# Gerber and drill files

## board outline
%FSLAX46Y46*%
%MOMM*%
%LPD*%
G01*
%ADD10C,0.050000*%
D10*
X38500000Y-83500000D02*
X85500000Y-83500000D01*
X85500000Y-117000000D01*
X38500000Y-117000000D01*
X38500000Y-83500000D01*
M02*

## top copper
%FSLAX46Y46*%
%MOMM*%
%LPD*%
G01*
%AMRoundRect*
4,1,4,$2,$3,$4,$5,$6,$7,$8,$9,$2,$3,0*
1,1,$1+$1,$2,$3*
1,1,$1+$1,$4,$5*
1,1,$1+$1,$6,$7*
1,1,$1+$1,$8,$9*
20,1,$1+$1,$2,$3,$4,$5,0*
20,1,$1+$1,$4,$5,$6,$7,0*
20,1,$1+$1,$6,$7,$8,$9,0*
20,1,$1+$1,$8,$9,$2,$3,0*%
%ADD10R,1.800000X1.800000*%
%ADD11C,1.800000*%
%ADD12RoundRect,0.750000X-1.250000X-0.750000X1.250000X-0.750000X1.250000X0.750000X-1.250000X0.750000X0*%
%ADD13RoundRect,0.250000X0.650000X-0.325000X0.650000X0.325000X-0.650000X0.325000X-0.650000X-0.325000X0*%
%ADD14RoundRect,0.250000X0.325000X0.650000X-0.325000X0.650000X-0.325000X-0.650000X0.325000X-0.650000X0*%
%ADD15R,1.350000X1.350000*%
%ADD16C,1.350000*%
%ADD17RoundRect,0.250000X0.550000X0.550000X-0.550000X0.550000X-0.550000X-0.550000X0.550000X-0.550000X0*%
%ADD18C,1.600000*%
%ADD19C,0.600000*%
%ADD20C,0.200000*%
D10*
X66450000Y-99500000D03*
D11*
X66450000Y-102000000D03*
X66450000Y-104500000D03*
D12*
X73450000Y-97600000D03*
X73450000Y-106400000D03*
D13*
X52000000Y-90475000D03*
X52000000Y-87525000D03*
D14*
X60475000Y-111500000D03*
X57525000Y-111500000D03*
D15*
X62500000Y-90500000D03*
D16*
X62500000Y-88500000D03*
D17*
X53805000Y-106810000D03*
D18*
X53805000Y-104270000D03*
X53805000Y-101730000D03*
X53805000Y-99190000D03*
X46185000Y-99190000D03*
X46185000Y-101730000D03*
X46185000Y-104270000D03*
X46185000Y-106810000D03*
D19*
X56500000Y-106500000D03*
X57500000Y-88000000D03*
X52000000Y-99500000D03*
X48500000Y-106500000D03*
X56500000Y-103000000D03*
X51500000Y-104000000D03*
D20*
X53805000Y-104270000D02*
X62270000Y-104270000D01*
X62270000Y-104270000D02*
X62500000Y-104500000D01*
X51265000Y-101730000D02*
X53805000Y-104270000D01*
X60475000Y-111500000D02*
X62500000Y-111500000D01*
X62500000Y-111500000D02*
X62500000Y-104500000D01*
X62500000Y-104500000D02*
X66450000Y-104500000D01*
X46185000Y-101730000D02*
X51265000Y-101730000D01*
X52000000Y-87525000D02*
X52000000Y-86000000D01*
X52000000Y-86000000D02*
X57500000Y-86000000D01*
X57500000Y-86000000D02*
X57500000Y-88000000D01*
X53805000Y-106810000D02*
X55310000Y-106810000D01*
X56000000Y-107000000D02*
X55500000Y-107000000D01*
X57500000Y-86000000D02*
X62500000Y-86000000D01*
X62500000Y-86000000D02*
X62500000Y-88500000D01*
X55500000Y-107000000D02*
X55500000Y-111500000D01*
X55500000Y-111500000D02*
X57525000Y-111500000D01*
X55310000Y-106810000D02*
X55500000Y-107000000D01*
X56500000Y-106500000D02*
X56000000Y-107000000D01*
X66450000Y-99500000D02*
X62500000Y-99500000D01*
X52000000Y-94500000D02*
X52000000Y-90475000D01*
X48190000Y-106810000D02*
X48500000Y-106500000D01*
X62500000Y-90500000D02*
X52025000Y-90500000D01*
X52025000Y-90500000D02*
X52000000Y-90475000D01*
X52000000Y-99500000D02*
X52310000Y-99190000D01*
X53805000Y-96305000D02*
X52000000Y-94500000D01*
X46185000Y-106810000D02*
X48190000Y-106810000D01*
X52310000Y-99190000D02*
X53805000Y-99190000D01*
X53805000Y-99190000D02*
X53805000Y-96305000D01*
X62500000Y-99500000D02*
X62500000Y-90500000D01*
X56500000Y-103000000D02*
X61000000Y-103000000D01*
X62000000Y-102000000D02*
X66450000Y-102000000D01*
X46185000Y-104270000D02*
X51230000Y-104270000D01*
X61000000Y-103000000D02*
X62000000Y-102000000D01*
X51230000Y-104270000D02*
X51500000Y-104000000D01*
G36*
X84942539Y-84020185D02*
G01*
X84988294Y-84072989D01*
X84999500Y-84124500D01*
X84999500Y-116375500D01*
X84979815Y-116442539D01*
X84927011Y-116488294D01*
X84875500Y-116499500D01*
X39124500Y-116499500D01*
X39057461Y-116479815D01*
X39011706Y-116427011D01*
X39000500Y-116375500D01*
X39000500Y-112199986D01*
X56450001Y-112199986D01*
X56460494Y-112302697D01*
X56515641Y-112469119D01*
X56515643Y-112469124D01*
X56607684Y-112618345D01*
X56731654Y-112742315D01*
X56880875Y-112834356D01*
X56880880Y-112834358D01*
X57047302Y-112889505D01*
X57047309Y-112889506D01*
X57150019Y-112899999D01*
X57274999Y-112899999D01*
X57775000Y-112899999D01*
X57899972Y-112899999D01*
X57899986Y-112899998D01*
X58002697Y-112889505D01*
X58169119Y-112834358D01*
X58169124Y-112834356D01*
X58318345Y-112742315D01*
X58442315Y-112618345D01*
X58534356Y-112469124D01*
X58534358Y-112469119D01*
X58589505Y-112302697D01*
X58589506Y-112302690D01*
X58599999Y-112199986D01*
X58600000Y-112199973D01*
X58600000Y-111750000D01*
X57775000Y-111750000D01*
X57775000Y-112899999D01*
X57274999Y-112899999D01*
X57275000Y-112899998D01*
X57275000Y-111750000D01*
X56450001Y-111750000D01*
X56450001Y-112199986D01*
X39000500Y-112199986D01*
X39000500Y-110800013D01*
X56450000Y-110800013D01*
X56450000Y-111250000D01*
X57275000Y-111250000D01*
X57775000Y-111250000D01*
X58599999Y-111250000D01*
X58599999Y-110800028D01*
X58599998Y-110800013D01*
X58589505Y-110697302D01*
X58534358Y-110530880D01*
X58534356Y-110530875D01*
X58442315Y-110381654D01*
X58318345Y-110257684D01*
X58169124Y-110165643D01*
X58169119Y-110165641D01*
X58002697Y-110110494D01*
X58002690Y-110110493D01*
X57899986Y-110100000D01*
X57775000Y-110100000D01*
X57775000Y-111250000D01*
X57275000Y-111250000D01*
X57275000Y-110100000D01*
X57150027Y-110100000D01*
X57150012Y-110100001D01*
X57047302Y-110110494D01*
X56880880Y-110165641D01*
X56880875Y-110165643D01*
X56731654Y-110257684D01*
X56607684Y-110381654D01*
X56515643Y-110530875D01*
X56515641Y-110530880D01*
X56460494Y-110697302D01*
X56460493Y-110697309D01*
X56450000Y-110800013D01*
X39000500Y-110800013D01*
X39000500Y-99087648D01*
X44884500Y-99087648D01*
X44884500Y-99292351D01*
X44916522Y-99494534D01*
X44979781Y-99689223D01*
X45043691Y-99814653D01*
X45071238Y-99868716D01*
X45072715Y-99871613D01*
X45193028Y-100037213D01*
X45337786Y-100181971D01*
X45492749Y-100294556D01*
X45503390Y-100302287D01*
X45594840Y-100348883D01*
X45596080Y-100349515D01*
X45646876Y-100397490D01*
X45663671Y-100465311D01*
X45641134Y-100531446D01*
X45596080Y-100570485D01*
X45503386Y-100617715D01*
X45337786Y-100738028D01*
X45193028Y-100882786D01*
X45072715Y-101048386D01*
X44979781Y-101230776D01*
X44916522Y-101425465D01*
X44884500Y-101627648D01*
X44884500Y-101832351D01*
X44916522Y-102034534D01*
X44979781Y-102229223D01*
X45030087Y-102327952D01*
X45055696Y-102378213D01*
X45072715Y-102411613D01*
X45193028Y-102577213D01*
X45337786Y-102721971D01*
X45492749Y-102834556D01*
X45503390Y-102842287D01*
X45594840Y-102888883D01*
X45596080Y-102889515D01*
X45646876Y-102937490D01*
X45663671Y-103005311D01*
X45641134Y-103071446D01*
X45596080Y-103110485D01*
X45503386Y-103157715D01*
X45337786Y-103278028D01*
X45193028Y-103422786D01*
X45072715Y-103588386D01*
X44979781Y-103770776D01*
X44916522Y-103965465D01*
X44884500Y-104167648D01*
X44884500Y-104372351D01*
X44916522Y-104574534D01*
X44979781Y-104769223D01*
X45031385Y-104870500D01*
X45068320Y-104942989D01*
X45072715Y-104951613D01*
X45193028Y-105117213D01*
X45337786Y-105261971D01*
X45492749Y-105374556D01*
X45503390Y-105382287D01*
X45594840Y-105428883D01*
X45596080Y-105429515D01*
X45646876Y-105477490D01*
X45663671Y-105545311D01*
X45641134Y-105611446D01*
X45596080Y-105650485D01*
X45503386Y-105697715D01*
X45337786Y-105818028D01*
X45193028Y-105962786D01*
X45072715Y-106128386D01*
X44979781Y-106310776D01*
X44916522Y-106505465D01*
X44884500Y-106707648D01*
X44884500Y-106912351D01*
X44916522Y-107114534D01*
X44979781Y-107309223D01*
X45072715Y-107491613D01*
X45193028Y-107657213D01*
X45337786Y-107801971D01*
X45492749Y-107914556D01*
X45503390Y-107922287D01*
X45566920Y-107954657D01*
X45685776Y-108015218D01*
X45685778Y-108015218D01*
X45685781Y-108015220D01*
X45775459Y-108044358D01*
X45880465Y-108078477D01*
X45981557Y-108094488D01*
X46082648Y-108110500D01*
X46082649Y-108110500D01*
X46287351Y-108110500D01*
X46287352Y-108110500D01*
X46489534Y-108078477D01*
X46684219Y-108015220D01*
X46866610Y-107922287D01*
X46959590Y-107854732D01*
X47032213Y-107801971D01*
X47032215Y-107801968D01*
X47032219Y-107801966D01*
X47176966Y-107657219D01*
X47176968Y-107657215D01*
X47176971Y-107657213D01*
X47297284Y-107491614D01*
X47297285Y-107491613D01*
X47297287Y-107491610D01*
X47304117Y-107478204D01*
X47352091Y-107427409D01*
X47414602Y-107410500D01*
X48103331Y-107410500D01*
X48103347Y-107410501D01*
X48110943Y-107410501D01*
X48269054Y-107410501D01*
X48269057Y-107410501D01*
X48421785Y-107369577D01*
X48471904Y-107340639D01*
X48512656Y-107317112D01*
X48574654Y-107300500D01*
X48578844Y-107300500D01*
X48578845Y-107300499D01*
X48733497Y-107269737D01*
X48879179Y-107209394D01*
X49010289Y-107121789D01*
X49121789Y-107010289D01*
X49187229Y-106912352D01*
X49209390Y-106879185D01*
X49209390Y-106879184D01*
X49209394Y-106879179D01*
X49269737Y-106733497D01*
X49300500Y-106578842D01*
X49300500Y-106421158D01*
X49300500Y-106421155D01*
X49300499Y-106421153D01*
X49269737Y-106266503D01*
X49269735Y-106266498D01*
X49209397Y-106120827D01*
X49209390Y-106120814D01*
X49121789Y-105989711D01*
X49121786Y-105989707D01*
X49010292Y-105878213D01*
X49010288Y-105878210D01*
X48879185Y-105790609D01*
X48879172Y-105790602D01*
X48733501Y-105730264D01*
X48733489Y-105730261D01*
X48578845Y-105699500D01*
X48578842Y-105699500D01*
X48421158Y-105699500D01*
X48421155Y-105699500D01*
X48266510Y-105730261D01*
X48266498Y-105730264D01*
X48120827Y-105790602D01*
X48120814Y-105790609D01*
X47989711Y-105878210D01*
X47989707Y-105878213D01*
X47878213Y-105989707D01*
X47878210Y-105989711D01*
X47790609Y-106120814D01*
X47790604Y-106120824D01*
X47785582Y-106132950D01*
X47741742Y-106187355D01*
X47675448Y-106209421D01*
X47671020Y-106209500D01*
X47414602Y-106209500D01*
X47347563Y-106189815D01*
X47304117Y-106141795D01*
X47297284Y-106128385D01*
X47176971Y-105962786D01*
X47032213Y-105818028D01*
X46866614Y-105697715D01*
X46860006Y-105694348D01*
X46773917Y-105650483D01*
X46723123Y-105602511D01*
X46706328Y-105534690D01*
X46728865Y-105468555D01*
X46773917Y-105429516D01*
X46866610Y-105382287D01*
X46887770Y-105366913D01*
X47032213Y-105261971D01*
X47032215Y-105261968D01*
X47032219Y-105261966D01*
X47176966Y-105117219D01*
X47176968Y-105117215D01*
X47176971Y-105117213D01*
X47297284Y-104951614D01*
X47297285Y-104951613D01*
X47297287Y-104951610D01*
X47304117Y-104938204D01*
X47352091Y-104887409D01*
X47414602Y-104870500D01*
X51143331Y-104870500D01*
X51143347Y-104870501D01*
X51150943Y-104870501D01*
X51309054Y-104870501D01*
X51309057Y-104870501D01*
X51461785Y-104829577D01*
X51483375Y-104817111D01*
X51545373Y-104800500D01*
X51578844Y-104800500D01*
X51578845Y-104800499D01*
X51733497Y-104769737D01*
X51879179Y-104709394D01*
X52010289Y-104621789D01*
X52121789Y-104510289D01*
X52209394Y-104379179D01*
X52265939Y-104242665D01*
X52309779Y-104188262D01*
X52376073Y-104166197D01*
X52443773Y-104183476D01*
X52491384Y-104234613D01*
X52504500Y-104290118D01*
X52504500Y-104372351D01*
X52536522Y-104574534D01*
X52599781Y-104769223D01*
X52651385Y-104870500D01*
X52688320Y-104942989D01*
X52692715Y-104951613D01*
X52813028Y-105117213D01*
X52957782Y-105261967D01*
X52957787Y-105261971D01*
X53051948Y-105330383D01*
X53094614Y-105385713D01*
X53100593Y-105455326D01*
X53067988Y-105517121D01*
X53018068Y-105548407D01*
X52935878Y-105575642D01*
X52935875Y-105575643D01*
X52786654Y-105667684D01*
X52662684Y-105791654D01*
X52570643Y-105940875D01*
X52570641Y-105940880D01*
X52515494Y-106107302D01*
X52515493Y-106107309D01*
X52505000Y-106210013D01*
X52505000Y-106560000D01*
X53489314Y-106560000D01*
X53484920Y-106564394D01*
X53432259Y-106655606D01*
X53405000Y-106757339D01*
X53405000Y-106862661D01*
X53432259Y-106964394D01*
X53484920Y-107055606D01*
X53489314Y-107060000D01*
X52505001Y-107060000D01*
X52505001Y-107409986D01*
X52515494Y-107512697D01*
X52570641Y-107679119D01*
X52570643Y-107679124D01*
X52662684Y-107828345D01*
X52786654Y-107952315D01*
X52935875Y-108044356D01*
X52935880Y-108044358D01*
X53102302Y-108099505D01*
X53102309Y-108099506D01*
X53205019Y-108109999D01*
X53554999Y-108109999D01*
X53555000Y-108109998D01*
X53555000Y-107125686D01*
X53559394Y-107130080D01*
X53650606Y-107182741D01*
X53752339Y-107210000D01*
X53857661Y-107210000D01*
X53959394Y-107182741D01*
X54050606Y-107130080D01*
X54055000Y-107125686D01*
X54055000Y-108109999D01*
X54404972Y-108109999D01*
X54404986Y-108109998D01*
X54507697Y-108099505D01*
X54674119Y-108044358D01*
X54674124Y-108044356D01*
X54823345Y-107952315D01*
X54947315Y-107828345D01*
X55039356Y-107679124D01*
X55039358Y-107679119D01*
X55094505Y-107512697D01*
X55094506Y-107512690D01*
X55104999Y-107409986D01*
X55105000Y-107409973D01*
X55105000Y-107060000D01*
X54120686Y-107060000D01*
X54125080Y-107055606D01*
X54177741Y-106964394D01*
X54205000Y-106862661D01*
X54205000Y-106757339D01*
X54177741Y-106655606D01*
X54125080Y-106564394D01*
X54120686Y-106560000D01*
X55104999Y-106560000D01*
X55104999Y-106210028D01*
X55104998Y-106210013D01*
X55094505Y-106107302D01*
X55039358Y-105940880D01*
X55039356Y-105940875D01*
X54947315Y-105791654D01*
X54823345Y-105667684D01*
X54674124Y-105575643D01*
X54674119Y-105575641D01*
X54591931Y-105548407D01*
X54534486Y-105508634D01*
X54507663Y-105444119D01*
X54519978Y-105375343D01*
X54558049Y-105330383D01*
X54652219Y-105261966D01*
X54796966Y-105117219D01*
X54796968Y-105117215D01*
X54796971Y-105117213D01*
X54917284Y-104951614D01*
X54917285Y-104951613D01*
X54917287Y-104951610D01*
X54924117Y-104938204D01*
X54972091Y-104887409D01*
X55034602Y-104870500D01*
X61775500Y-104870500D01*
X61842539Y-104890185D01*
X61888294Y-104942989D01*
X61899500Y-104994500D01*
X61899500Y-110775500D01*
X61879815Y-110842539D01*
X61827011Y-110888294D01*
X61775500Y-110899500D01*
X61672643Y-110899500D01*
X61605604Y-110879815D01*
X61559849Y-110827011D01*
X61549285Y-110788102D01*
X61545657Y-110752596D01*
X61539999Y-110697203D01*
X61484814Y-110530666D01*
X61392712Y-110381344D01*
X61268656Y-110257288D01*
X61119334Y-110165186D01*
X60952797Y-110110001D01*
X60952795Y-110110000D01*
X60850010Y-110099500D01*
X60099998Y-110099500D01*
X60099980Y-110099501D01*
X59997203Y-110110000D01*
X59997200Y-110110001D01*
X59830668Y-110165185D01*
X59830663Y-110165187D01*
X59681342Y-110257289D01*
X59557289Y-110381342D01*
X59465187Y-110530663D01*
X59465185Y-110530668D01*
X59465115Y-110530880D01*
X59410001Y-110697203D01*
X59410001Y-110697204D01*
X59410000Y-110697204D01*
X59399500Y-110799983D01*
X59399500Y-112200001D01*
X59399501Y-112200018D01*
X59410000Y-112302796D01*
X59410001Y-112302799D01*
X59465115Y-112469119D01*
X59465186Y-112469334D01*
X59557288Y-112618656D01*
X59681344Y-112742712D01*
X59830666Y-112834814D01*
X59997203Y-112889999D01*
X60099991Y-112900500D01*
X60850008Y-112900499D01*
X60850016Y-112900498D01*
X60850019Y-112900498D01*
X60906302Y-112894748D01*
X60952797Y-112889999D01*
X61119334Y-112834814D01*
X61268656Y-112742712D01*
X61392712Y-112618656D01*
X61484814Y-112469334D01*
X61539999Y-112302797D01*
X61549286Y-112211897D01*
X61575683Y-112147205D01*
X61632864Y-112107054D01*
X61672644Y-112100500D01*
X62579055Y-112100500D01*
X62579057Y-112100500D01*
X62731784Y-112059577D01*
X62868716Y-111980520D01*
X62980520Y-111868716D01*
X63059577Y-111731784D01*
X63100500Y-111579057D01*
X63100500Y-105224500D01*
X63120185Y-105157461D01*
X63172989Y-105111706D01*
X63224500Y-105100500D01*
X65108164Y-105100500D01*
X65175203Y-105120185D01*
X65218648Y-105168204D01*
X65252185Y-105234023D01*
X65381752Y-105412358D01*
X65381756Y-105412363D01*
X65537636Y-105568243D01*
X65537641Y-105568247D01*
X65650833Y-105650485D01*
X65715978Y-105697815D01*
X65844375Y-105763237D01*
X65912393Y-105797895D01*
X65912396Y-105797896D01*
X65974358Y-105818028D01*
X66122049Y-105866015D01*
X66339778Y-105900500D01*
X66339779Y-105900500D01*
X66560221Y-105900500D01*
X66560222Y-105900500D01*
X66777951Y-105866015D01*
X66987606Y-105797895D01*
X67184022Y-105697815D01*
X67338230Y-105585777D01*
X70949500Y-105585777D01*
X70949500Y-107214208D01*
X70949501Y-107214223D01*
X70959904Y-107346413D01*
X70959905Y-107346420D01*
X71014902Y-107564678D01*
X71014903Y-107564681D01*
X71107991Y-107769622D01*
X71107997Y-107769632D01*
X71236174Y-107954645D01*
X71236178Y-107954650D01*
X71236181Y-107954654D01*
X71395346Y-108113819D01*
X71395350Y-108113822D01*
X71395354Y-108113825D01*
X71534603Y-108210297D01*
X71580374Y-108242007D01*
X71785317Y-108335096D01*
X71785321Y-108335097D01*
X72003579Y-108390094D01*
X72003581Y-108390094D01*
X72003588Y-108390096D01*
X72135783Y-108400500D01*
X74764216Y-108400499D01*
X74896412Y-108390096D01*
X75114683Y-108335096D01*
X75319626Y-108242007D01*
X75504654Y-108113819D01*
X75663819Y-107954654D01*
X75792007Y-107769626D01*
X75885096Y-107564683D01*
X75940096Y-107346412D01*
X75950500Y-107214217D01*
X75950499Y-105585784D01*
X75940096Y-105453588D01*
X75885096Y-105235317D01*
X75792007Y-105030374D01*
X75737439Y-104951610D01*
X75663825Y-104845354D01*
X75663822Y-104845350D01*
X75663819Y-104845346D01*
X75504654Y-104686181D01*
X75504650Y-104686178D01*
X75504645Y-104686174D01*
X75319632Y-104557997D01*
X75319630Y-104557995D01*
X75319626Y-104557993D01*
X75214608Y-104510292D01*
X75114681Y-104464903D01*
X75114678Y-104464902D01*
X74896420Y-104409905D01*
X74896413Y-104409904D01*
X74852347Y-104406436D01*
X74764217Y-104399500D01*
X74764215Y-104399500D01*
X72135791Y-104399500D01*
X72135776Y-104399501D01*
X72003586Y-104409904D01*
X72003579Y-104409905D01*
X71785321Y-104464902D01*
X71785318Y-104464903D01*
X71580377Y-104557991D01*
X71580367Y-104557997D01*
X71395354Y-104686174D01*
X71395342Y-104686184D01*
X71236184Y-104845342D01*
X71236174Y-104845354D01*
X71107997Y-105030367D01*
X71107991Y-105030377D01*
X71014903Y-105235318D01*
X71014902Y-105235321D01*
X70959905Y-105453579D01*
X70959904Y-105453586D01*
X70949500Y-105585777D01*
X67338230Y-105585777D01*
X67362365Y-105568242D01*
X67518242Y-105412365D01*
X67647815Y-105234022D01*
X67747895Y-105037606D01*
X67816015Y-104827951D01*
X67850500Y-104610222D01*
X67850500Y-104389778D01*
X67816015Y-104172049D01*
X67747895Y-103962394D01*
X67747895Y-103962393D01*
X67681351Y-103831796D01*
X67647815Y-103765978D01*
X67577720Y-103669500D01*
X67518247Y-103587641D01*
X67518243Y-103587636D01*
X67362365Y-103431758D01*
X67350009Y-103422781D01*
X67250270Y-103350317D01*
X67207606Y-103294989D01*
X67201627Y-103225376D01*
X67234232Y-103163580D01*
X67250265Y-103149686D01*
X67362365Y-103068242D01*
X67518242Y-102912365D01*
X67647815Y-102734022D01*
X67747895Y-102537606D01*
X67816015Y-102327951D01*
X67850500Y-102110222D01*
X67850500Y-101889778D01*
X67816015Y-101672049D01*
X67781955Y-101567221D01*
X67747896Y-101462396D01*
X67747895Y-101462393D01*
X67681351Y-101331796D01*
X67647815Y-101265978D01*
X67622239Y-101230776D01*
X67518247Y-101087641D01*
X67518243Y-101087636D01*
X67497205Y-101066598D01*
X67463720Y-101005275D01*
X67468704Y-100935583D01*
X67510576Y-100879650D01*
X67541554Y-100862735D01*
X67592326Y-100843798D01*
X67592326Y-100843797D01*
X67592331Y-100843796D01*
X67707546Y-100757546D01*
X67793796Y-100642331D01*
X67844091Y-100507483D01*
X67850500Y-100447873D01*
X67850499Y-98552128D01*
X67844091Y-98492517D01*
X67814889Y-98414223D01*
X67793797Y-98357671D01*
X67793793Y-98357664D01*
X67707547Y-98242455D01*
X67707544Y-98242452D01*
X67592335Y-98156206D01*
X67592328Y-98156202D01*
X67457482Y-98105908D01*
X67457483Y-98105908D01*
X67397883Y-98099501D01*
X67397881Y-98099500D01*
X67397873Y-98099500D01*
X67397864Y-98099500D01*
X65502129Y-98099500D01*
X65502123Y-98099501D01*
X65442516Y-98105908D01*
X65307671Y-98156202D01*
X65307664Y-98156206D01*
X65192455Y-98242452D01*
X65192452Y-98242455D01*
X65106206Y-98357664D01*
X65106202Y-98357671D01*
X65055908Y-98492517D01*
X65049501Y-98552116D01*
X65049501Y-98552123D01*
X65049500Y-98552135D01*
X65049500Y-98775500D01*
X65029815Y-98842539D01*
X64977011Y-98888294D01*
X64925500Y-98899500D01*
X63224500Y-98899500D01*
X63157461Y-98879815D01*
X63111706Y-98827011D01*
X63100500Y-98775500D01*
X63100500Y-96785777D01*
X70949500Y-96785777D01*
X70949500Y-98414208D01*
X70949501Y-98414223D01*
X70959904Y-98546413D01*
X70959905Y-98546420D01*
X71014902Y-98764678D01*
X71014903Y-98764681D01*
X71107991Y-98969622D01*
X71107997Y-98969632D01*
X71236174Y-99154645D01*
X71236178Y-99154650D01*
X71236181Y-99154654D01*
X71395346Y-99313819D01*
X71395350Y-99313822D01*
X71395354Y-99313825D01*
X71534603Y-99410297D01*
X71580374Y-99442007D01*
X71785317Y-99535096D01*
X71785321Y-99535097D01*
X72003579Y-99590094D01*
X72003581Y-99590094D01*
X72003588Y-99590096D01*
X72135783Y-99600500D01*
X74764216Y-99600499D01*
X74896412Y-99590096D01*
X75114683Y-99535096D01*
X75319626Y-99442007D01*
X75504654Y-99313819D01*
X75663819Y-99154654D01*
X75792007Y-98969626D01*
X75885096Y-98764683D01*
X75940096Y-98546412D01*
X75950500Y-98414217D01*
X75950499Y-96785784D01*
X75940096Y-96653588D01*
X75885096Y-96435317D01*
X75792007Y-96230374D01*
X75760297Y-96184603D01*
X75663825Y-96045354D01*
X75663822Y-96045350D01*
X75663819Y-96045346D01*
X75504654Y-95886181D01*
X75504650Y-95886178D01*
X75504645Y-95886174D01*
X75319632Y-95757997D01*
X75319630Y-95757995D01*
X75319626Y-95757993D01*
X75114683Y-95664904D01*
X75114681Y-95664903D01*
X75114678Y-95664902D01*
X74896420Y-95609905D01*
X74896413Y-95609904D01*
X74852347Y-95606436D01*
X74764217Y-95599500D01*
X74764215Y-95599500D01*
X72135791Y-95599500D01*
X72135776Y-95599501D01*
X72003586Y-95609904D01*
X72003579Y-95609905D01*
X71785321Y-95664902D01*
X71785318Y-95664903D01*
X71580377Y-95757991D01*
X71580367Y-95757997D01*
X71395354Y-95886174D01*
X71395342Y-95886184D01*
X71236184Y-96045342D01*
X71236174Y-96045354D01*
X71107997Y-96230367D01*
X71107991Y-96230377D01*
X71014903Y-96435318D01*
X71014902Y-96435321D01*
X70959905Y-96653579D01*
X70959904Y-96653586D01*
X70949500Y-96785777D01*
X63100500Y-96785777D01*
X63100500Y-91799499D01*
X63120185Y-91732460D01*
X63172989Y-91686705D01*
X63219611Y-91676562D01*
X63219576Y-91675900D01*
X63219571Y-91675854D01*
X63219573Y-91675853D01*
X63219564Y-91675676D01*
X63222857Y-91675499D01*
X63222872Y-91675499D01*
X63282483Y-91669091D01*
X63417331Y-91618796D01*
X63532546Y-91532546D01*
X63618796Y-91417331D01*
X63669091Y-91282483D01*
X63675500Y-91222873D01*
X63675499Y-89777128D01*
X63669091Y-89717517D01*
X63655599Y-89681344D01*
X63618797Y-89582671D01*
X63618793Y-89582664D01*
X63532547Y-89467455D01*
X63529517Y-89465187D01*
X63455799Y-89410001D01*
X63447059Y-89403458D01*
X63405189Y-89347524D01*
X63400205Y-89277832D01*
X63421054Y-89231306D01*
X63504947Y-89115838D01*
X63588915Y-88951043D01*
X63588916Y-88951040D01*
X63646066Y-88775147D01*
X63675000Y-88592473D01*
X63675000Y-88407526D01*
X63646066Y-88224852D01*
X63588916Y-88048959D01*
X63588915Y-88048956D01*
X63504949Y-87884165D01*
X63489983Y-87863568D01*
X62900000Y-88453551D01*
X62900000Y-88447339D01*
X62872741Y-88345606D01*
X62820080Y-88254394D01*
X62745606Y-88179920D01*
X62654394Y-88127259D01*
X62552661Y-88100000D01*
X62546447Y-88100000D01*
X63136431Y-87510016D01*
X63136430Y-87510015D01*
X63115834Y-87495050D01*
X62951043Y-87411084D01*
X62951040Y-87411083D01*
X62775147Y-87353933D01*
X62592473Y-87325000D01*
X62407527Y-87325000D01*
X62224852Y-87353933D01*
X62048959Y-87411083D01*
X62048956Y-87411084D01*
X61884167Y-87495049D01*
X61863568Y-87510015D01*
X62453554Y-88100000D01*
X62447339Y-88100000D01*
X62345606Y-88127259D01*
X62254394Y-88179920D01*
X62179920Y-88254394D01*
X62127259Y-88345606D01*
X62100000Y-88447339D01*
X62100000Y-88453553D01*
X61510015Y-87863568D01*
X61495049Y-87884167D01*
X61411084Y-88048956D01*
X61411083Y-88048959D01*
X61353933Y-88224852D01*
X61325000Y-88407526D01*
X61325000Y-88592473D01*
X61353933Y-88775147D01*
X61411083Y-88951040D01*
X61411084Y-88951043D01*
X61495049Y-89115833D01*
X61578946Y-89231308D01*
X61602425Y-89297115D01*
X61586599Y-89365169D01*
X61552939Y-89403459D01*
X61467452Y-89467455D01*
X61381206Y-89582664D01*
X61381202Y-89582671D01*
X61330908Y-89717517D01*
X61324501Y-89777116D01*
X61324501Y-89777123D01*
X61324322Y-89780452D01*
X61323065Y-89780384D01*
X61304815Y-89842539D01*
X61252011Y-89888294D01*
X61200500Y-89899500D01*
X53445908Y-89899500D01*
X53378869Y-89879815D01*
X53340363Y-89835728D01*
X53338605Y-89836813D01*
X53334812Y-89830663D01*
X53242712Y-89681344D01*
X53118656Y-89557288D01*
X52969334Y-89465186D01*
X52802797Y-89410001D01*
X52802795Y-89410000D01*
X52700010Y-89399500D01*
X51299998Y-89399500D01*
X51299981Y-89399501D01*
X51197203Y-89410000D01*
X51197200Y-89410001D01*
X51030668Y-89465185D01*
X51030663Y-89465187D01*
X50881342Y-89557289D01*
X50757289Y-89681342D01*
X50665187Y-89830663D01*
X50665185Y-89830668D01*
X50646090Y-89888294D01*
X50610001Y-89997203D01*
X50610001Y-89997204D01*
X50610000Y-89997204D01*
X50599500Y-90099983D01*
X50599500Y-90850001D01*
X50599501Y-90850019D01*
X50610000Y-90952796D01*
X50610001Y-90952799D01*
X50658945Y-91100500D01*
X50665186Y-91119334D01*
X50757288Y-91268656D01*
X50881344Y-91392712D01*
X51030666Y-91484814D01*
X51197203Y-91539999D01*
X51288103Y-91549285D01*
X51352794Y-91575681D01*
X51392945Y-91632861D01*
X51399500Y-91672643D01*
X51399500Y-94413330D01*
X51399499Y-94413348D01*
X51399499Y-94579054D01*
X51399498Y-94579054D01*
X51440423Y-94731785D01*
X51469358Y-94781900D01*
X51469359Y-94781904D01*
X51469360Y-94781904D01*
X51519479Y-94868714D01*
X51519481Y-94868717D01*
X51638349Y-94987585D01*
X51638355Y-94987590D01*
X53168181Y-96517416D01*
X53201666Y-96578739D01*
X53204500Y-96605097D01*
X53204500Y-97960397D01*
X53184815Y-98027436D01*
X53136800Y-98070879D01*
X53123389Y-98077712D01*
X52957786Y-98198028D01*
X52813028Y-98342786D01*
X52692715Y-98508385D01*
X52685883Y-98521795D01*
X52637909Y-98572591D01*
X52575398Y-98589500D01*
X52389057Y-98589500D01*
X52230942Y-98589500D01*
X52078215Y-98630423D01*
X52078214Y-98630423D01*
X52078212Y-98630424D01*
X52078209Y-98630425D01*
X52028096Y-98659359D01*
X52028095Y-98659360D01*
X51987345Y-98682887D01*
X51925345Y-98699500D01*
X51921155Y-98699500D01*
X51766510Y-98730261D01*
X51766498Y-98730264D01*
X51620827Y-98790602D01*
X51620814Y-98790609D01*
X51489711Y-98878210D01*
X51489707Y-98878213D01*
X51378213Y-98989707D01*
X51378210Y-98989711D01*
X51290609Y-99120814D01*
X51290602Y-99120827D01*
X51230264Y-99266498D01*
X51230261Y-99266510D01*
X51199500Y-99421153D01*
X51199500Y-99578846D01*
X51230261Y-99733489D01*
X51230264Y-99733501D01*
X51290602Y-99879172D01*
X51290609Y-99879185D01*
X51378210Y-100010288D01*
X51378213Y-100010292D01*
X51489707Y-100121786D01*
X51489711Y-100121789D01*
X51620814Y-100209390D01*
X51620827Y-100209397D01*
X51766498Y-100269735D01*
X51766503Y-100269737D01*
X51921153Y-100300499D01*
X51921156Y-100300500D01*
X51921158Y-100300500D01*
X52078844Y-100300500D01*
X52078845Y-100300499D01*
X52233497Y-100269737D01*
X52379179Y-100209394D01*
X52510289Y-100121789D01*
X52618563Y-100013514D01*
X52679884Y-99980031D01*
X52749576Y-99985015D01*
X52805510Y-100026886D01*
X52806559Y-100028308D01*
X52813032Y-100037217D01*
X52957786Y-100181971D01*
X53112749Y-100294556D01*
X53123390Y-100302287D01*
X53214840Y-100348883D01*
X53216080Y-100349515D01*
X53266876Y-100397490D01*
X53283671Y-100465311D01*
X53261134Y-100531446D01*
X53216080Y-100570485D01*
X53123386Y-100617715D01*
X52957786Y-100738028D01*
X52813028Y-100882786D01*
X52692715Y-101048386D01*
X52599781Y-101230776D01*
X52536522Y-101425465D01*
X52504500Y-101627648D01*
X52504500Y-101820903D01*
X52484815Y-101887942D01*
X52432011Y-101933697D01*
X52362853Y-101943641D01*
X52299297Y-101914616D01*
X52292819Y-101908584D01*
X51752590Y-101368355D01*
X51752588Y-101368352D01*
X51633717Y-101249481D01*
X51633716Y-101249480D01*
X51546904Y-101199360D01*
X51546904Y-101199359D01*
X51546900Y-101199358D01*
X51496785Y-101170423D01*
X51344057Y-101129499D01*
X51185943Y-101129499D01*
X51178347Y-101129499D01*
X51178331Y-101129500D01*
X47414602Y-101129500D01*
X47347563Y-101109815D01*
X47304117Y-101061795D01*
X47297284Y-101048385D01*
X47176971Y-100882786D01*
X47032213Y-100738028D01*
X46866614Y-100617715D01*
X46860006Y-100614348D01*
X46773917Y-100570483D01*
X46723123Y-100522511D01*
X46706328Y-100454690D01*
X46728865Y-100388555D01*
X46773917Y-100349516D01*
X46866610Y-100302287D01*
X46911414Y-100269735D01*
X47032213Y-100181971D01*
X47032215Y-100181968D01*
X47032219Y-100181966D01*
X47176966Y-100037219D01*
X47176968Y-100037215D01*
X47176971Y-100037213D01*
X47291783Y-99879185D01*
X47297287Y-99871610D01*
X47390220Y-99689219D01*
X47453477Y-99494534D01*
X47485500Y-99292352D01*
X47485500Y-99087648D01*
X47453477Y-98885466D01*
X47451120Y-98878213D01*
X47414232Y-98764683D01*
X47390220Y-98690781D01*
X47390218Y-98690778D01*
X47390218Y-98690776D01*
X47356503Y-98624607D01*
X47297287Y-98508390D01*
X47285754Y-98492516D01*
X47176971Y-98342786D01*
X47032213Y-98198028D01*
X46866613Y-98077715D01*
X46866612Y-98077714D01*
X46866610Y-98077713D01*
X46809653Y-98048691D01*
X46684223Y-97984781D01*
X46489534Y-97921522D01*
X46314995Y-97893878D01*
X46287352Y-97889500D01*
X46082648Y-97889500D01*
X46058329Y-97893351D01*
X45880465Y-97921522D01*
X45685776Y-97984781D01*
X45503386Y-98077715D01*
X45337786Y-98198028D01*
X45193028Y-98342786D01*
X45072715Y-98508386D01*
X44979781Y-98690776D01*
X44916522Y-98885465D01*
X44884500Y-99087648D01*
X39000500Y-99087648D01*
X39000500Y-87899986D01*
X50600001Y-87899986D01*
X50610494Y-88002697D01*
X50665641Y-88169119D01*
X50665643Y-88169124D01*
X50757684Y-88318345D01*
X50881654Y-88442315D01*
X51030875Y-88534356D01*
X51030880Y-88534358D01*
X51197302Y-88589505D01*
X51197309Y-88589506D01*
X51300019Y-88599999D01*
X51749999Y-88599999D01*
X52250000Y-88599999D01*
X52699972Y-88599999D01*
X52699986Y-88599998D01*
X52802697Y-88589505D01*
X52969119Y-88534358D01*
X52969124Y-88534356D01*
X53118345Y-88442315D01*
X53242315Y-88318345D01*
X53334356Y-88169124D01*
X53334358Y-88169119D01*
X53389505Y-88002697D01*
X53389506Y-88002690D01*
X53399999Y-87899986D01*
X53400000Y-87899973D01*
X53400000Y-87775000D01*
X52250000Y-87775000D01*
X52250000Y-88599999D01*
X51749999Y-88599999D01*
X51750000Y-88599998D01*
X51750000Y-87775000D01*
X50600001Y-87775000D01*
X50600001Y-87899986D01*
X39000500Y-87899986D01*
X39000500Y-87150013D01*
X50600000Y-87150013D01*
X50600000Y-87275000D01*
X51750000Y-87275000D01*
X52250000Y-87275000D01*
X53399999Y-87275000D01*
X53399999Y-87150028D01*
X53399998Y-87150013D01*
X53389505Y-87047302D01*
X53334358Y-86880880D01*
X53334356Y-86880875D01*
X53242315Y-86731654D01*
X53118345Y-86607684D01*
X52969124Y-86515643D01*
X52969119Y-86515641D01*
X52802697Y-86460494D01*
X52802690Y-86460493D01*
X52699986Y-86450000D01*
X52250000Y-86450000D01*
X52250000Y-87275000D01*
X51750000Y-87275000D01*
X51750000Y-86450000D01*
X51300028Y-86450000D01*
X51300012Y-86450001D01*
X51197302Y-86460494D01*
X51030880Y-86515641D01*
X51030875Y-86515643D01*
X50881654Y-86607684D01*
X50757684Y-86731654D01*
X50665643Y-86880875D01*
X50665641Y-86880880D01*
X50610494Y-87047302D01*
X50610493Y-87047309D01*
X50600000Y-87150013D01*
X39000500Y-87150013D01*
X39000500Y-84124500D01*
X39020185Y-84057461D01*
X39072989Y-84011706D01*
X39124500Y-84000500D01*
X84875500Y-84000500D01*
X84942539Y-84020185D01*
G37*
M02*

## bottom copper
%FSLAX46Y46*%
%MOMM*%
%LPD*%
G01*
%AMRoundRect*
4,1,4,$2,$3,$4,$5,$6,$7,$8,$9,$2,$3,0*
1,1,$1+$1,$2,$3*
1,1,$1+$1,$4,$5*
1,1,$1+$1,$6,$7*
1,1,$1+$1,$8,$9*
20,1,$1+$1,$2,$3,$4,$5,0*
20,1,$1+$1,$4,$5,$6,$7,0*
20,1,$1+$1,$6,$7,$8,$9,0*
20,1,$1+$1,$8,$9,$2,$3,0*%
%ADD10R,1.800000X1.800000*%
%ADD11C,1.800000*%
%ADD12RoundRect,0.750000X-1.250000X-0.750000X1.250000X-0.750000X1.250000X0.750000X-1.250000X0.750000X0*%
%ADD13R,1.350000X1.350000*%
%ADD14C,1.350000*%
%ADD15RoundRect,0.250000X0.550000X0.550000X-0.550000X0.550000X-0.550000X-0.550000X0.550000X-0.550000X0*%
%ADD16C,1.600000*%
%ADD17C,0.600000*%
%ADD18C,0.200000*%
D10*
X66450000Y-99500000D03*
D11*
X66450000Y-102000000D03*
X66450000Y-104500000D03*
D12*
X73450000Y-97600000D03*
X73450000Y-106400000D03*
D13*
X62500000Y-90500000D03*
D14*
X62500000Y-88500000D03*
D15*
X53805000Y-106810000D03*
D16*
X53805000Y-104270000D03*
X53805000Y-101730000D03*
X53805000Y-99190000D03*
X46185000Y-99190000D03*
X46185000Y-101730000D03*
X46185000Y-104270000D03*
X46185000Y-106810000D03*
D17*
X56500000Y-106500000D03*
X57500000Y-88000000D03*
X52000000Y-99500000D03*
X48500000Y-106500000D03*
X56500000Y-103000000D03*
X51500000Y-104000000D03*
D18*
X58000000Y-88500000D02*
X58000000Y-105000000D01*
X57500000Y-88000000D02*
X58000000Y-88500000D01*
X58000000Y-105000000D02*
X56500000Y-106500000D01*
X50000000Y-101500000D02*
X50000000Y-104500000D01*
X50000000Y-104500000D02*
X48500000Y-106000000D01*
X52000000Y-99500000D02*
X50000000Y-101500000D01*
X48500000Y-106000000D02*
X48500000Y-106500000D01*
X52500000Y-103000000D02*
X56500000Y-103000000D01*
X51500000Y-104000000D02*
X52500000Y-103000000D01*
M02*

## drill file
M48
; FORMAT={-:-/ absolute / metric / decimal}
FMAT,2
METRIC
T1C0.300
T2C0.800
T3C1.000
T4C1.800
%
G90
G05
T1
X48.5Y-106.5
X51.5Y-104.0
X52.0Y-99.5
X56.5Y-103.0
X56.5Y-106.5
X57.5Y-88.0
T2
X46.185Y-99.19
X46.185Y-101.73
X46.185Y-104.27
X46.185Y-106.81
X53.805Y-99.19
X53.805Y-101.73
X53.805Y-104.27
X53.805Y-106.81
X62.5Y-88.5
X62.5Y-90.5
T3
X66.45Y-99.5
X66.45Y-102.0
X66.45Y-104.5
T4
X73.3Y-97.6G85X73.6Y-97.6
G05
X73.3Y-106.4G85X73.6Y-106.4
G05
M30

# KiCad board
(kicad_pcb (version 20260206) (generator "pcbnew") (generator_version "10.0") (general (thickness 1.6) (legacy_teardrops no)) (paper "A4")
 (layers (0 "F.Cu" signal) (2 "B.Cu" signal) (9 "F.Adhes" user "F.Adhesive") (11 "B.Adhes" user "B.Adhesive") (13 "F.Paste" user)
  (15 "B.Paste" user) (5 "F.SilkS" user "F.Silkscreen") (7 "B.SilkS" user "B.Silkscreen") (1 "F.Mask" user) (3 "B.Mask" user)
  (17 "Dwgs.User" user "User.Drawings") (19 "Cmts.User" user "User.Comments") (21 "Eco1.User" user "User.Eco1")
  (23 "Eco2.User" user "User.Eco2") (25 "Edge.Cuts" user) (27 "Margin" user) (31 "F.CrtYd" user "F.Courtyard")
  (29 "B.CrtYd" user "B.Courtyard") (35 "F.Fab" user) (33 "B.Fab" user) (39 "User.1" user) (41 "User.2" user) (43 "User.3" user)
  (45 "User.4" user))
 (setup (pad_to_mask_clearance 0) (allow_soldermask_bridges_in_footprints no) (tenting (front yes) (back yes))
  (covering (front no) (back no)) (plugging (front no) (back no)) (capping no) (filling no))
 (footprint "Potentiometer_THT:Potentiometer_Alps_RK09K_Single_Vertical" (layer "F.Cu") (at 66.45 99.5)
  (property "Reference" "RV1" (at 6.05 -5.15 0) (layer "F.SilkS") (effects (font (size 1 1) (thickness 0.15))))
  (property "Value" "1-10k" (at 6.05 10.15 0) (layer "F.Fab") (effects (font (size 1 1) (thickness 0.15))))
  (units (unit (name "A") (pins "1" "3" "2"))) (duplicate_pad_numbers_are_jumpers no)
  (pad "1" thru_hole rect (at 0 0) (size 1.8 1.8) (drill 1) (layers "*.Cu" "*.Mask") (remove_unused_layers no) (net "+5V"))
  (pad "2" thru_hole circle (at 0 2.5) (size 1.8 1.8) (drill 1) (layers "*.Cu" "*.Mask") (remove_unused_layers no) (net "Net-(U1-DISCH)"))
  (pad "3" thru_hole circle (at 0 5) (size 1.8 1.8) (drill 1) (layers "*.Cu" "*.Mask") (remove_unused_layers no) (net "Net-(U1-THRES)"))
  (pad "MP" thru_hole roundrect (at 7 -1.9) (size 4 3) (drill oval 2.1 1.8) (layers "*.Cu" "*.Mask") (remove_unused_layers no)
   (roundrect_rratio 0.25))
  (pad "MP" thru_hole roundrect (at 7 6.9) (size 4 3) (drill oval 2.1 1.8) (layers "*.Cu" "*.Mask") (remove_unused_layers no)
   (roundrect_rratio 0.25)))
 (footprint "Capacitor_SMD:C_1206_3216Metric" (layer "F.Cu") (at 52 89 90)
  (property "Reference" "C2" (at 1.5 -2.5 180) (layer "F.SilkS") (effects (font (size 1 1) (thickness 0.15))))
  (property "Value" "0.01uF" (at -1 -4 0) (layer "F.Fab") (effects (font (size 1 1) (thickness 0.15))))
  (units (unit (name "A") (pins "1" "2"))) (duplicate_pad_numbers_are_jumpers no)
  (pad "1" smd roundrect (at -1.475 0 90) (size 1.15 1.8) (layers "F.Cu" "F.Mask" "F.Paste") (roundrect_rratio 0.217391) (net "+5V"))
  (pad "2" smd roundrect (at 1.475 0 90) (size 1.15 1.8) (layers "F.Cu" "F.Mask" "F.Paste") (roundrect_rratio 0.217391) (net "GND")))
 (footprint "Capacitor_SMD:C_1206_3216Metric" (layer "F.Cu") (at 59 111.5 180)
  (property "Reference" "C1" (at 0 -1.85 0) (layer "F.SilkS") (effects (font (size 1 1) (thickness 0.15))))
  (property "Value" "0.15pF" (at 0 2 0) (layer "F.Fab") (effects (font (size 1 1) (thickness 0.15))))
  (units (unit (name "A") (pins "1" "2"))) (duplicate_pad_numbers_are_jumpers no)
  (pad "1" smd roundrect (at -1.475 0 180) (size 1.15 1.8) (layers "F.Cu" "F.Mask" "F.Paste") (roundrect_rratio 0.217391)
   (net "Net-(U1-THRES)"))
  (pad "2" smd roundrect (at 1.475 0 180) (size 1.15 1.8) (layers "F.Cu" "F.Mask" "F.Paste") (roundrect_rratio 0.217391) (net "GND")))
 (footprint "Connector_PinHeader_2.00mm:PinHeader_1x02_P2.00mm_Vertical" (layer "F.Cu") (at 62.5 90.5 180)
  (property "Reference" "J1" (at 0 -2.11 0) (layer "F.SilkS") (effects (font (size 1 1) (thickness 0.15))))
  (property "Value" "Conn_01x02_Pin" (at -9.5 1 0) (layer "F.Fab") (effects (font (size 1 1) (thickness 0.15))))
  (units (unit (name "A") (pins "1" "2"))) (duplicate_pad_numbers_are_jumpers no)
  (pad "1" thru_hole rect (at 0 0 180) (size 1.35 1.35) (drill 0.8) (layers "*.Cu" "*.Mask") (remove_unused_layers no) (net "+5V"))
  (pad "2" thru_hole circle (at 0 2 180) (size 1.35 1.35) (drill 0.8) (layers "*.Cu" "*.Mask") (remove_unused_layers no) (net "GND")))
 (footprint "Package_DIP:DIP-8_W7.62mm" (layer "F.Cu") (at 53.805 106.81 180)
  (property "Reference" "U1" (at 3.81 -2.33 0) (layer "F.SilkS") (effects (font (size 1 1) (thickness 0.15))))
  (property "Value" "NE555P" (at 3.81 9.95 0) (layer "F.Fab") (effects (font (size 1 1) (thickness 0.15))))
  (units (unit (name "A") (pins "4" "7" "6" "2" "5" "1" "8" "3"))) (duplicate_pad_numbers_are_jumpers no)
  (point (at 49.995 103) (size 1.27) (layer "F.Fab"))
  (pad "1" thru_hole roundrect (at 0 0 180) (size 1.6 1.6) (drill 0.8) (layers "*.Cu" "*.Mask") (remove_unused_layers no)
   (roundrect_rratio 0.15625) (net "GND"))
  (pad "2" thru_hole circle (at 0 2.54 180) (size 1.6 1.6) (drill 0.8) (layers "*.Cu" "*.Mask") (remove_unused_layers no)
   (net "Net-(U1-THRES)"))
  (pad "3" thru_hole circle (at 0 5.08 180) (size 1.6 1.6) (drill 0.8) (layers "*.Cu" "*.Mask") (remove_unused_layers no)
   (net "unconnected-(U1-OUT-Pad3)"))
  (pad "4" thru_hole circle (at 0 7.62 180) (size 1.6 1.6) (drill 0.8) (layers "*.Cu" "*.Mask") (remove_unused_layers no) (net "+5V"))
  (pad "5" thru_hole circle (at 7.62 7.62 180) (size 1.6 1.6) (drill 0.8) (layers "*.Cu" "*.Mask") (remove_unused_layers no)
   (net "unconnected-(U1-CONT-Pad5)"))
  (pad "6" thru_hole circle (at 7.62 5.08 180) (size 1.6 1.6) (drill 0.8) (layers "*.Cu" "*.Mask") (remove_unused_layers no)
   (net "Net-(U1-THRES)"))
  (pad "7" thru_hole circle (at 7.62 2.54 180) (size 1.6 1.6) (drill 0.8) (layers "*.Cu" "*.Mask") (remove_unused_layers no)
   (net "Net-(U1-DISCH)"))
  (pad "8" thru_hole circle (at 7.62 0 180) (size 1.6 1.6) (drill 0.8) (layers "*.Cu" "*.Mask") (remove_unused_layers no) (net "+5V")))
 (gr_rect (start 38.5 83.5) (end 85.5 117) (stroke (width 0.05) (type default)) (fill no) (layer "Edge.Cuts"))
 (segment (start 53.805 104.27) (end 62.27 104.27) (width 0.2) (layer "F.Cu") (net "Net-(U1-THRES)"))
 (segment (start 62.27 104.27) (end 62.5 104.5) (width 0.2) (layer "F.Cu") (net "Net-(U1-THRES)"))
 (segment (start 51.265 101.73) (end 53.805 104.27) (width 0.2) (layer "F.Cu") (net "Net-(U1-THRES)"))
 (segment (start 60.475 111.5) (end 62.5 111.5) (width 0.2) (layer "F.Cu") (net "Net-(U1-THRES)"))
 (segment (start 62.5 111.5) (end 62.5 104.5) (width 0.2) (layer "F.Cu") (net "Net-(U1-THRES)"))
 (segment (start 62.5 104.5) (end 66.45 104.5) (width 0.2) (layer "F.Cu") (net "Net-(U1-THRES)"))
 (segment (start 46.185 101.73) (end 51.265 101.73) (width 0.2) (layer "F.Cu") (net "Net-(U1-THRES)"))
 (segment (start 52 87.525) (end 52 86) (width 0.2) (layer "F.Cu") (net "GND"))
 (segment (start 52 86) (end 57.5 86) (width 0.2) (layer "F.Cu") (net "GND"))
 (segment (start 57.5 86) (end 57.5 88) (width 0.2) (layer "F.Cu") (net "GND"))
 (segment (start 53.805 106.81) (end 55.31 106.81) (width 0.2) (layer "F.Cu") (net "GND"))
 (segment (start 56 107) (end 55.5 107) (width 0.2) (layer "F.Cu") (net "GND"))
 (segment (start 57.5 86) (end 62.5 86) (width 0.2) (layer "F.Cu") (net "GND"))
 (segment (start 62.5 86) (end 62.5 88.5) (width 0.2) (layer "F.Cu") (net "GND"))
 (segment (start 55.5 107) (end 55.5 111.5) (width 0.2) (layer "F.Cu") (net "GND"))
 (segment (start 55.5 111.5) (end 57.525 111.5) (width 0.2) (layer "F.Cu") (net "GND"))
 (segment (start 55.31 106.81) (end 55.5 107) (width 0.2) (layer "F.Cu") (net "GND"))
 (segment (start 56.5 106.5) (end 56 107) (width 0.2) (layer "F.Cu") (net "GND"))
 (via (at 56.5 106.5) (size 0.6) (drill 0.3) (layers "F.Cu" "B.Cu") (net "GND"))
 (via (at 57.5 88) (size 0.6) (drill 0.3) (layers "F.Cu" "B.Cu") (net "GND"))
 (segment (start 58 88.5) (end 58 105) (width 0.2) (layer "B.Cu") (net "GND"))
 (segment (start 57.5 88) (end 58 88.5) (width 0.2) (layer "B.Cu") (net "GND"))
 (segment (start 58 105) (end 56.5 106.5) (width 0.2) (layer "B.Cu") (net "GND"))
 (segment (start 66.45 99.5) (end 62.5 99.5) (width 0.2) (layer "F.Cu") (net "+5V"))
 (segment (start 52 94.5) (end 52 90.475) (width 0.2) (layer "F.Cu") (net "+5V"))
 (segment (start 48.19 106.81) (end 48.5 106.5) (width 0.2) (layer "F.Cu") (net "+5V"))
 (segment (start 62.5 90.5) (end 52.025 90.5) (width 0.2) (layer "F.Cu") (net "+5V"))
 (segment (start 52.025 90.5) (end 52 90.475) (width 0.2) (layer "F.Cu") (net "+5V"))
 (segment (start 52 99.5) (end 52.31 99.19) (width 0.2) (layer "F.Cu") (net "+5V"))
 (segment (start 53.805 96.305) (end 52 94.5) (width 0.2) (layer "F.Cu") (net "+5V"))
 (segment (start 46.185 106.81) (end 48.19 106.81) (width 0.2) (layer "F.Cu") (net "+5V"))
 (segment (start 52.31 99.19) (end 53.805 99.19) (width 0.2) (layer "F.Cu") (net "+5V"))
 (segment (start 53.805 99.19) (end 53.805 96.305) (width 0.2) (layer "F.Cu") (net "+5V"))
 (segment (start 62.5 99.5) (end 62.5 90.5) (width 0.2) (layer "F.Cu") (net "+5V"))
 (via (at 52 99.5) (size 0.6) (drill 0.3) (layers "F.Cu" "B.Cu") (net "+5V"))
 (via (at 48.5 106.5) (size 0.6) (drill 0.3) (layers "F.Cu" "B.Cu") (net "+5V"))
 (segment (start 50 101.5) (end 50 104.5) (width 0.2) (layer "B.Cu") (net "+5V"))
 (segment (start 50 104.5) (end 48.5 106) (width 0.2) (layer "B.Cu") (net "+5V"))
 (segment (start 52 99.5) (end 50 101.5) (width 0.2) (layer "B.Cu") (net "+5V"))
 (segment (start 48.5 106) (end 48.5 106.5) (width 0.2) (layer "B.Cu") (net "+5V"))
 (segment (start 56.5 103) (end 61 103) (width 0.2) (layer "F.Cu") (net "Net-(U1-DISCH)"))
 (segment (start 62 102) (end 66.45 102) (width 0.2) (layer "F.Cu") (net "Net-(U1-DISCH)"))
 (segment (start 46.185 104.27) (end 51.23 104.27) (width 0.2) (layer "F.Cu") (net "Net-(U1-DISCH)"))
 (segment (start 61 103) (end 62 102) (width 0.2) (layer "F.Cu") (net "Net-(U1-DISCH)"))
 (segment (start 51.23 104.27) (end 51.5 104) (width 0.2) (layer "F.Cu") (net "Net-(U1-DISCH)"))
 (via (at 56.5 103) (size 0.6) (drill 0.3) (layers "F.Cu" "B.Cu") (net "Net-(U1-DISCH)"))
 (via (at 51.5 104) (size 0.6) (drill 0.3) (layers "F.Cu" "B.Cu") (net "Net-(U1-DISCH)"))
 (segment (start 52.5 103) (end 56.5 103) (width 0.2) (layer "B.Cu") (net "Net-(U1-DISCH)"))
 (segment (start 51.5 104) (end 52.5 103) (width 0.2) (layer "B.Cu") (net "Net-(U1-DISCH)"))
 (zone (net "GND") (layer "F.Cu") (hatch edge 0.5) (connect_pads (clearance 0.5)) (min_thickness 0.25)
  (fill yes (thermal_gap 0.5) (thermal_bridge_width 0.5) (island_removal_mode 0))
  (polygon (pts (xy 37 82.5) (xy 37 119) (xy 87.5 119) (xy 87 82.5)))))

